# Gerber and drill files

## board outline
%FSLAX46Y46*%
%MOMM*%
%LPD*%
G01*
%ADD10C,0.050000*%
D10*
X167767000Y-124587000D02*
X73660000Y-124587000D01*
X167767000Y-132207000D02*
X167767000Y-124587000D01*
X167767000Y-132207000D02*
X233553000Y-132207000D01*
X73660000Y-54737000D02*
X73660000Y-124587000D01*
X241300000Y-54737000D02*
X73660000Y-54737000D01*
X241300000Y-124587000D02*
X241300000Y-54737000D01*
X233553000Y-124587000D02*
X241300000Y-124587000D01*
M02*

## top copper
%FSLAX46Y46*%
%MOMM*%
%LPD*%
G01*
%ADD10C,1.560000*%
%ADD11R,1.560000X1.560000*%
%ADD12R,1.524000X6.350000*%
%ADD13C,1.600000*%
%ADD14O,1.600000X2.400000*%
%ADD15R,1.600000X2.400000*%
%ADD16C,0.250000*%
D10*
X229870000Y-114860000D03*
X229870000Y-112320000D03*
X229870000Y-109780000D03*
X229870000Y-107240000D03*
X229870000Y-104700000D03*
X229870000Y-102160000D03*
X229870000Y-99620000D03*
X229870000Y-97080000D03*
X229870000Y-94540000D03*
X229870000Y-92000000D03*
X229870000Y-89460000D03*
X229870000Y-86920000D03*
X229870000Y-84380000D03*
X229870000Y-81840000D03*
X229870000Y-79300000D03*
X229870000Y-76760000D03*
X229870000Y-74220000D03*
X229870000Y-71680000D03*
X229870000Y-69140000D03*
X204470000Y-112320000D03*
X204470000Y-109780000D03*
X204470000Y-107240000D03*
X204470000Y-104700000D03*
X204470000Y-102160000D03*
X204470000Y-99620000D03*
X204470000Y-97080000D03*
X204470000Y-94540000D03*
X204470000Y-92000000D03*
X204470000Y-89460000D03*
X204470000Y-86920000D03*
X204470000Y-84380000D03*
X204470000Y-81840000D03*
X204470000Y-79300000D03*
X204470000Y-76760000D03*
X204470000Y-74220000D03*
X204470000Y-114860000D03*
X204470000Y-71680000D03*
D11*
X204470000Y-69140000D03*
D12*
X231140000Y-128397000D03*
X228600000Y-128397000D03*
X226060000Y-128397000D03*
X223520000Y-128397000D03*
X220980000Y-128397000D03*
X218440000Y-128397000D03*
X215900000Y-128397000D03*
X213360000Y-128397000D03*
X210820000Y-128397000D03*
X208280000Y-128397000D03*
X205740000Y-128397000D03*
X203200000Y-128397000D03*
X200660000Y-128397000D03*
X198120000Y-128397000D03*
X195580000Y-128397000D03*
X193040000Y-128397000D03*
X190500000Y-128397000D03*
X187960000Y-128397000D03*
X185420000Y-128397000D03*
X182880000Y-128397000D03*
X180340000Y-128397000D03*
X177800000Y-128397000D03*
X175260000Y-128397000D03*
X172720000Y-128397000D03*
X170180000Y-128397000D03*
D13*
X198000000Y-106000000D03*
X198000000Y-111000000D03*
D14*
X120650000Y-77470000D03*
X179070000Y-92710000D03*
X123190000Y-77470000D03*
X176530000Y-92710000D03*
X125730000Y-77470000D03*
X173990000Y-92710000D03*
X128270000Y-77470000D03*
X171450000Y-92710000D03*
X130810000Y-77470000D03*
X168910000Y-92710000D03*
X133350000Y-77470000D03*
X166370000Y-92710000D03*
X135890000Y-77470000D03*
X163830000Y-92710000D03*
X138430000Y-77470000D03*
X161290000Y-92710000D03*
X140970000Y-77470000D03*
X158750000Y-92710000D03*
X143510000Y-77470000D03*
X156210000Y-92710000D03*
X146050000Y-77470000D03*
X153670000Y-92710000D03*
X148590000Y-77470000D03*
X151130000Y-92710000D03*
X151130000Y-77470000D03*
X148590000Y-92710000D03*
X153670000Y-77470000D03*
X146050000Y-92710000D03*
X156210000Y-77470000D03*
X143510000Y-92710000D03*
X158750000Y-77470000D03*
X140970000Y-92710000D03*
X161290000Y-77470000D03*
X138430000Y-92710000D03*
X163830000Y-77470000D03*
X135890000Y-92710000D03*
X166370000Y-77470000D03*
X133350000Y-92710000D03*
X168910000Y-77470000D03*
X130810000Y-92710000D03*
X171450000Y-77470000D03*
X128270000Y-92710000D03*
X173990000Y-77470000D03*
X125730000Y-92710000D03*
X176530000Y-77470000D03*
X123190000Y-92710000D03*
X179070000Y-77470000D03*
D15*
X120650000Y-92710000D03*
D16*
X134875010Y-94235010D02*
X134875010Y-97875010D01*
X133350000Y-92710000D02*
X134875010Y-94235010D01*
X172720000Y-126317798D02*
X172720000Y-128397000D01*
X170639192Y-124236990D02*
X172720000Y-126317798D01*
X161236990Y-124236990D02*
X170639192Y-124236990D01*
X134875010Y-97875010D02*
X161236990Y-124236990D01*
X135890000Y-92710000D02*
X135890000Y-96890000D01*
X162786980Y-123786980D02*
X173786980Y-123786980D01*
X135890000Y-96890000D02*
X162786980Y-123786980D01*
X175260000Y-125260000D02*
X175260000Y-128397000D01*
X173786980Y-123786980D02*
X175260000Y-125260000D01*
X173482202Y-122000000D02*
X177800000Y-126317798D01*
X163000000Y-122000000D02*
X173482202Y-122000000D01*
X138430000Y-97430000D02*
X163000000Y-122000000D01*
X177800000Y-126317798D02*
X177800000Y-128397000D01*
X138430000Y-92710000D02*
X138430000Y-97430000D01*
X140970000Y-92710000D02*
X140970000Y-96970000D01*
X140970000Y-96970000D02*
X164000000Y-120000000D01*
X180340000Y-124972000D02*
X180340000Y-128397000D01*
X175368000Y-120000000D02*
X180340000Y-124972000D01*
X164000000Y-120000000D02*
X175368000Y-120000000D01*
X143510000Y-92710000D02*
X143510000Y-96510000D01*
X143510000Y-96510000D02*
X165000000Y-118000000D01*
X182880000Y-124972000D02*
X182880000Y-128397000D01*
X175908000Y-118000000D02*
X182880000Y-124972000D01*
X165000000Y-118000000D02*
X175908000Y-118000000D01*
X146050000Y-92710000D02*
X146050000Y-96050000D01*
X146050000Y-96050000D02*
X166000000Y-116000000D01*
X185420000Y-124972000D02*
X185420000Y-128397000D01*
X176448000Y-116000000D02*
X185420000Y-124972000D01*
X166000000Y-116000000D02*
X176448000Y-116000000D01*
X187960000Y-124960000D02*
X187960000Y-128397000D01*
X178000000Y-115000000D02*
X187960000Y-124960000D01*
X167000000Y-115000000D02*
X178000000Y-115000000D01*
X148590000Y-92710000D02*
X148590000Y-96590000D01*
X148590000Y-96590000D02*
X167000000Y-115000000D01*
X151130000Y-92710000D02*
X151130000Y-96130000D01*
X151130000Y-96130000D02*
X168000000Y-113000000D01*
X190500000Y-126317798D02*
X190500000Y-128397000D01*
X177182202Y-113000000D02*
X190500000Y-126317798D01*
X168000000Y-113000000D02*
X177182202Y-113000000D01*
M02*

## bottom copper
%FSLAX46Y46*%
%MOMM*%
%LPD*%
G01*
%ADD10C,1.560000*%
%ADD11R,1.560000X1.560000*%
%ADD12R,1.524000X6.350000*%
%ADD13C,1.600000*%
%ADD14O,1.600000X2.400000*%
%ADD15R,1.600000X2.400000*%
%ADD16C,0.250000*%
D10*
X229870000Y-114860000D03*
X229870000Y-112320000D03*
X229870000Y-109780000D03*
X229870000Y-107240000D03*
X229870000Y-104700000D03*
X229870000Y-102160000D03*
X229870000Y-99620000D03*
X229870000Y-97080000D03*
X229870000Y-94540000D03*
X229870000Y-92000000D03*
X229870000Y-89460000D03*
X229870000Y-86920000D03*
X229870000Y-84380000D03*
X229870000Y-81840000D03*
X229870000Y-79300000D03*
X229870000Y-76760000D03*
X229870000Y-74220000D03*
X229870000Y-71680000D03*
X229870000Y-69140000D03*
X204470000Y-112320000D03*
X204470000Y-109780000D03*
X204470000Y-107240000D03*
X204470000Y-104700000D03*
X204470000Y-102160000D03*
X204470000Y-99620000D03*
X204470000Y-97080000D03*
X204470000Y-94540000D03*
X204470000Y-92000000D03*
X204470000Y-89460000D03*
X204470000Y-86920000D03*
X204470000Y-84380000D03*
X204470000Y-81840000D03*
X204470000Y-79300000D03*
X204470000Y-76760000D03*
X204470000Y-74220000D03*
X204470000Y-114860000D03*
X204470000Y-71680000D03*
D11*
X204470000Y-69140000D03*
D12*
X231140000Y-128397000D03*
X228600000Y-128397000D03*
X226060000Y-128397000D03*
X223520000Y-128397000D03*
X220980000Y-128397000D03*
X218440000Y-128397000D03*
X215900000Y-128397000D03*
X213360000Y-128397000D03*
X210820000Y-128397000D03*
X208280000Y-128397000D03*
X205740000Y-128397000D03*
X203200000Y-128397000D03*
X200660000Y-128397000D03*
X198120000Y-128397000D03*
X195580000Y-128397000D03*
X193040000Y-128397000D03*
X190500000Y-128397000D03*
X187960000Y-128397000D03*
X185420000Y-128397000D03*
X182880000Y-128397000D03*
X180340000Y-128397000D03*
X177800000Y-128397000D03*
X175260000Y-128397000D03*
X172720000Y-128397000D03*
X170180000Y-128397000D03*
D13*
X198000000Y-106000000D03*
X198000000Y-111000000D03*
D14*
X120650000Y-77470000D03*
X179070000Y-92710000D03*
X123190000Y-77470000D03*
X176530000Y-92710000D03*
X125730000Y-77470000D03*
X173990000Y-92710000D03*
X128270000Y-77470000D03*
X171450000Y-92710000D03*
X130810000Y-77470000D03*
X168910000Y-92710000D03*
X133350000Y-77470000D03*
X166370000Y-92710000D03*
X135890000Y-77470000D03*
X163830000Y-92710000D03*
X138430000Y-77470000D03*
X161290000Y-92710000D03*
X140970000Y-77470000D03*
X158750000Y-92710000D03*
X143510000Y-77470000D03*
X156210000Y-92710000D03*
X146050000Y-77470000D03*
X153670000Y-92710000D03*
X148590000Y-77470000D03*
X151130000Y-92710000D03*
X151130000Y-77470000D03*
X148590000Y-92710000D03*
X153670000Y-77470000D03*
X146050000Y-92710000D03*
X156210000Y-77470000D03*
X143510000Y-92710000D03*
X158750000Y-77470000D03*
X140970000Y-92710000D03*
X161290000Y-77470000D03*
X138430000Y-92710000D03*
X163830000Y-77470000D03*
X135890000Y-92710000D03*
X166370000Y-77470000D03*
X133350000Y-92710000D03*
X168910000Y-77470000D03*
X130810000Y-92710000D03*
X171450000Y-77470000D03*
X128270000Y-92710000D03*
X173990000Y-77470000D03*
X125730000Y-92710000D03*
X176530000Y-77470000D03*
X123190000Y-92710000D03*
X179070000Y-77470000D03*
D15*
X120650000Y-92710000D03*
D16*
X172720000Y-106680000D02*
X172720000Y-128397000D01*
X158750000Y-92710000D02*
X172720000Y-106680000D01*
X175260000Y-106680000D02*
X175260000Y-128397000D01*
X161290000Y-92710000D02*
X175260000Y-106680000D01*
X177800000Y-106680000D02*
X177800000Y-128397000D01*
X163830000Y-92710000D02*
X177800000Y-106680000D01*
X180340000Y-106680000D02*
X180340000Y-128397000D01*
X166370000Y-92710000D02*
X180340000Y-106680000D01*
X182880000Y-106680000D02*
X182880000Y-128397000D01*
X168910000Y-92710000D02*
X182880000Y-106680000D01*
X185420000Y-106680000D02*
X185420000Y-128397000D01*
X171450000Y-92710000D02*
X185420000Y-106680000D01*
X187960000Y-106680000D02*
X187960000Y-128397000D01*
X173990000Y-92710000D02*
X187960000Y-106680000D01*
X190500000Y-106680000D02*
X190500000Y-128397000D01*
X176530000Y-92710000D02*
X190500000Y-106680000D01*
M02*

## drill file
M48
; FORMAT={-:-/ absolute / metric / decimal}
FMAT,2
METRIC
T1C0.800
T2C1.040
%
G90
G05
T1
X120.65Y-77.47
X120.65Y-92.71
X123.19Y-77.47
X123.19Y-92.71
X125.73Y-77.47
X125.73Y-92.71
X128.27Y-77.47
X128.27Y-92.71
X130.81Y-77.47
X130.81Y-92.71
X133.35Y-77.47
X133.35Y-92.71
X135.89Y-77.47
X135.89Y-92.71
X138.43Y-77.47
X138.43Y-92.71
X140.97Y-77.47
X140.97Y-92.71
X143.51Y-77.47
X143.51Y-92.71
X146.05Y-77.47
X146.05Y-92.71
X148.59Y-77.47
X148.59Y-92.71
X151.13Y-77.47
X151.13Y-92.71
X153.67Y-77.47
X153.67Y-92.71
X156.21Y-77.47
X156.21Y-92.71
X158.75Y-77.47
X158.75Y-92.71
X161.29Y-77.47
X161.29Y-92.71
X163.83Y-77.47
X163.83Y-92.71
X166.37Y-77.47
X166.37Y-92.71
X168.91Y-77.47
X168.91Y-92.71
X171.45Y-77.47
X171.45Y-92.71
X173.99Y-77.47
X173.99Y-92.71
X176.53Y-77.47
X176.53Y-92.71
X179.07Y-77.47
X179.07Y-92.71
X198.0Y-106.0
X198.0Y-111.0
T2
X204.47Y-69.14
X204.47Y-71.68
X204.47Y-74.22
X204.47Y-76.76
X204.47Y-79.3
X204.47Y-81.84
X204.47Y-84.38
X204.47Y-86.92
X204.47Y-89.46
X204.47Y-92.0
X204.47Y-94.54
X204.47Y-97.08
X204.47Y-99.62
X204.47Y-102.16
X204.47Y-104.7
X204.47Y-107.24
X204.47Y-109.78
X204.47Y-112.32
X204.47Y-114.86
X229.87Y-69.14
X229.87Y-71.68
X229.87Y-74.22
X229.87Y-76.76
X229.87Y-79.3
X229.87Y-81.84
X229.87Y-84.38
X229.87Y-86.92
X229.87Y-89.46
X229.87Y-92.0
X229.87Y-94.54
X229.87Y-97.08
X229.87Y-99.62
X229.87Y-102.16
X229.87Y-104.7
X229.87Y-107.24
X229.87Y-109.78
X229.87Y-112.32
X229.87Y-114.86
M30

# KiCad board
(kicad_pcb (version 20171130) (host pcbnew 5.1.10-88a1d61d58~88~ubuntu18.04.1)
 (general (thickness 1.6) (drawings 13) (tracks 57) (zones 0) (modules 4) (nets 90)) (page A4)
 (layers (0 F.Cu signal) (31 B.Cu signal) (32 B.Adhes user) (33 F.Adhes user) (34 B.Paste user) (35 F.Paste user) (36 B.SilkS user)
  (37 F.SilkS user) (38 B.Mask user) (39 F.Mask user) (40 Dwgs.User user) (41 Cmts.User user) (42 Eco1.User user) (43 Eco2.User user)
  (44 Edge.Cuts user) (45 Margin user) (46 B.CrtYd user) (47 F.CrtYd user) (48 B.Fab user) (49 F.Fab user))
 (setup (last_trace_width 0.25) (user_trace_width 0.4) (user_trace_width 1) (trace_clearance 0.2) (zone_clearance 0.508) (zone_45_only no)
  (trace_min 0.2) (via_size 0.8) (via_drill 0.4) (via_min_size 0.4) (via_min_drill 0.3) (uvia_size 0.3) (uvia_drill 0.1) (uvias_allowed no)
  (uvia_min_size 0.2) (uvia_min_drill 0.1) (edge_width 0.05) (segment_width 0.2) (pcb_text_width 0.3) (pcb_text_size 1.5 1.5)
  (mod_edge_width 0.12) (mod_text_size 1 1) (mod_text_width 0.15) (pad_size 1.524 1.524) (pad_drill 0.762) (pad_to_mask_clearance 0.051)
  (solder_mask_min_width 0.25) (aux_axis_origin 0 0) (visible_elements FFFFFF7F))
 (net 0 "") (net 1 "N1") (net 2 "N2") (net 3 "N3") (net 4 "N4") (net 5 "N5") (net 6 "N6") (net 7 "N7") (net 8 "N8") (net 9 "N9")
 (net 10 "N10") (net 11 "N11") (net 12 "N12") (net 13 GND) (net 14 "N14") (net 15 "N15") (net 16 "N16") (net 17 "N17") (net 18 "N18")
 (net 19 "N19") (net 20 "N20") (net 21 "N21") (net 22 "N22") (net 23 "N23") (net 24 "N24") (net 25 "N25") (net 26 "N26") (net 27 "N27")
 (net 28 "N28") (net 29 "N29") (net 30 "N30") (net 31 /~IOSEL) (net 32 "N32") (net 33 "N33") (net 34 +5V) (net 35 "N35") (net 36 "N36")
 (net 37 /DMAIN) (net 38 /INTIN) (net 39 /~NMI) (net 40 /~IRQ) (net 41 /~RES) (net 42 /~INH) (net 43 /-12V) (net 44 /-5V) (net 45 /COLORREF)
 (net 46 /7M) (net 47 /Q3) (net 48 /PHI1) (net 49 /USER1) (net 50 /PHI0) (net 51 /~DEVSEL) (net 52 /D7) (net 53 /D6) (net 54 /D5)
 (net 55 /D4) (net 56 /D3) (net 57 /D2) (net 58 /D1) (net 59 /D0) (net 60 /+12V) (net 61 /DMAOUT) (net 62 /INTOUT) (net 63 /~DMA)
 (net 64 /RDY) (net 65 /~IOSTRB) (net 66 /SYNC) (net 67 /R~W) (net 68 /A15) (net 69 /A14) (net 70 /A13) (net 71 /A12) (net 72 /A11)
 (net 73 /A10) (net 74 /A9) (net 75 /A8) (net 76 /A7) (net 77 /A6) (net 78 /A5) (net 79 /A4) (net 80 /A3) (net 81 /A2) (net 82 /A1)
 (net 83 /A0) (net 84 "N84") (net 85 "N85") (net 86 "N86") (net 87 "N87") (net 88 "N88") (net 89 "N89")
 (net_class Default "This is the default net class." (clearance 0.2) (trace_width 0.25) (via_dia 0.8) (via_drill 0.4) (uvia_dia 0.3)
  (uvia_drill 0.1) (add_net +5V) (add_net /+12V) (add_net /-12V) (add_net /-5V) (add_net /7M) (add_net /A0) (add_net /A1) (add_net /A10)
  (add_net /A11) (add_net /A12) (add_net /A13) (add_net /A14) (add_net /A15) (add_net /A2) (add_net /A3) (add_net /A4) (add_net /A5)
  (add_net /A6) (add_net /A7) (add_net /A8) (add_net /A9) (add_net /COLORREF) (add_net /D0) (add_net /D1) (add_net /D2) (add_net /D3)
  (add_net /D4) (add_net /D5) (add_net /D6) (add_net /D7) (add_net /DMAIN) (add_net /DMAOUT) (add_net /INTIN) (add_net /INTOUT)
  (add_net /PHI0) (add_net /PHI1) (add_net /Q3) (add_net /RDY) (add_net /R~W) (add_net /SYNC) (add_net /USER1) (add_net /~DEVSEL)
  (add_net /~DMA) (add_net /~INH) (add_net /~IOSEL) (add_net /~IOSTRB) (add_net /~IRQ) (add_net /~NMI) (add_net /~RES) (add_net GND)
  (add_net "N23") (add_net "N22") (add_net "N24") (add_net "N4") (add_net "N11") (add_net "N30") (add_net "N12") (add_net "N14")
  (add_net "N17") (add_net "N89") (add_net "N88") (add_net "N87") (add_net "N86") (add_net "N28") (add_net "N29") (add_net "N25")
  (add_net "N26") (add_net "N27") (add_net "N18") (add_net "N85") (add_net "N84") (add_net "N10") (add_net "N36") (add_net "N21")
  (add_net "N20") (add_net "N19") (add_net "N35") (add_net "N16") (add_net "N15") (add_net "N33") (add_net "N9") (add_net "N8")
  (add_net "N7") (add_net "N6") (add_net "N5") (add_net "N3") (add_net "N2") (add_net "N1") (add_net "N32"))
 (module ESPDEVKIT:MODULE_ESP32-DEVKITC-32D (layer F.Cu) (at 217.17 88.9)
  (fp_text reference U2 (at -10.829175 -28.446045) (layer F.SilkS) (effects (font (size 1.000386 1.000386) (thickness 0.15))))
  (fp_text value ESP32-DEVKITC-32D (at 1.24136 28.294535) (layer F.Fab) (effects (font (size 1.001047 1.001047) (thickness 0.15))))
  (pad 38 thru_hole circle (at 12.7 25.96) (size 1.56 1.56) (drill 1.04) (layers *.Cu *.Mask) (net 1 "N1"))
  (pad 37 thru_hole circle (at 12.7 23.42) (size 1.56 1.56) (drill 1.04) (layers *.Cu *.Mask) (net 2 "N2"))
  (pad 36 thru_hole circle (at 12.7 20.88) (size 1.56 1.56) (drill 1.04) (layers *.Cu *.Mask) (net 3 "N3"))
  (pad 35 thru_hole circle (at 12.7 18.34) (size 1.56 1.56) (drill 1.04) (layers *.Cu *.Mask) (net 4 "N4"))
  (pad 34 thru_hole circle (at 12.7 15.8) (size 1.56 1.56) (drill 1.04) (layers *.Cu *.Mask) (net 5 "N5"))
  (pad 33 thru_hole circle (at 12.7 13.26) (size 1.56 1.56) (drill 1.04) (layers *.Cu *.Mask) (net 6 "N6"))
  (pad 32 thru_hole circle (at 12.7 10.72) (size 1.56 1.56) (drill 1.04) (layers *.Cu *.Mask) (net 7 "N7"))
  (pad 31 thru_hole circle (at 12.7 8.18) (size 1.56 1.56) (drill 1.04) (layers *.Cu *.Mask) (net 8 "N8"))
  (pad 30 thru_hole circle (at 12.7 5.64) (size 1.56 1.56) (drill 1.04) (layers *.Cu *.Mask) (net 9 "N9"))
  (pad 29 thru_hole circle (at 12.7 3.1) (size 1.56 1.56) (drill 1.04) (layers *.Cu *.Mask) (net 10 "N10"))
  (pad 28 thru_hole circle (at 12.7 0.56) (size 1.56 1.56) (drill 1.04) (layers *.Cu *.Mask) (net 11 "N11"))
  (pad 27 thru_hole circle (at 12.7 -1.98) (size 1.56 1.56) (drill 1.04) (layers *.Cu *.Mask) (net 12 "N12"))
  (pad 26 thru_hole circle (at 12.7 -4.52) (size 1.56 1.56) (drill 1.04) (layers *.Cu *.Mask) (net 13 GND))
  (pad 25 thru_hole circle (at 12.7 -7.06) (size 1.56 1.56) (drill 1.04) (layers *.Cu *.Mask) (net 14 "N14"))
  (pad 24 thru_hole circle (at 12.7 -9.6) (size 1.56 1.56) (drill 1.04) (layers *.Cu *.Mask) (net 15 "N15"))
  (pad 23 thru_hole circle (at 12.7 -12.14) (size 1.56 1.56) (drill 1.04) (layers *.Cu *.Mask) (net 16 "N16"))
  (pad 22 thru_hole circle (at 12.7 -14.68) (size 1.56 1.56) (drill 1.04) (layers *.Cu *.Mask) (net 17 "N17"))
  (pad 21 thru_hole circle (at 12.7 -17.22) (size 1.56 1.56) (drill 1.04) (layers *.Cu *.Mask) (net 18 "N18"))
  (pad 20 thru_hole circle (at 12.7 -19.76) (size 1.56 1.56) (drill 1.04) (layers *.Cu *.Mask) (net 13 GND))
  (pad 18 thru_hole circle (at -12.7 23.42) (size 1.56 1.56) (drill 1.04) (layers *.Cu *.Mask) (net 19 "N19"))
  (pad 17 thru_hole circle (at -12.7 20.88) (size 1.56 1.56) (drill 1.04) (layers *.Cu *.Mask) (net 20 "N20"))
  (pad 16 thru_hole circle (at -12.7 18.34) (size 1.56 1.56) (drill 1.04) (layers *.Cu *.Mask) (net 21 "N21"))
  (pad 15 thru_hole circle (at -12.7 15.8) (size 1.56 1.56) (drill 1.04) (layers *.Cu *.Mask) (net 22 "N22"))
  (pad 14 thru_hole circle (at -12.7 13.26) (size 1.56 1.56) (drill 1.04) (layers *.Cu *.Mask) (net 13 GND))
  (pad 13 thru_hole circle (at -12.7 10.72) (size 1.56 1.56) (drill 1.04) (layers *.Cu *.Mask) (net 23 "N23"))
  (pad 12 thru_hole circle (at -12.7 8.18) (size 1.56 1.56) (drill 1.04) (layers *.Cu *.Mask) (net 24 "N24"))
  (pad 11 thru_hole circle (at -12.7 5.64) (size 1.56 1.56) (drill 1.04) (layers *.Cu *.Mask) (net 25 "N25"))
  (pad 10 thru_hole circle (at -12.7 3.1) (size 1.56 1.56) (drill 1.04) (layers *.Cu *.Mask) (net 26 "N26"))
  (pad 9 thru_hole circle (at -12.7 0.56) (size 1.56 1.56) (drill 1.04) (layers *.Cu *.Mask) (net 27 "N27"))
  (pad 8 thru_hole circle (at -12.7 -1.98) (size 1.56 1.56) (drill 1.04) (layers *.Cu *.Mask) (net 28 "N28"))
  (pad 7 thru_hole circle (at -12.7 -4.52) (size 1.56 1.56) (drill 1.04) (layers *.Cu *.Mask) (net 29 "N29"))
  (pad 6 thru_hole circle (at -12.7 -7.06) (size 1.56 1.56) (drill 1.04) (layers *.Cu *.Mask) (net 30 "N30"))
  (pad 5 thru_hole circle (at -12.7 -9.6) (size 1.56 1.56) (drill 1.04) (layers *.Cu *.Mask) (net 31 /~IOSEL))
  (pad 4 thru_hole circle (at -12.7 -12.14) (size 1.56 1.56) (drill 1.04) (layers *.Cu *.Mask) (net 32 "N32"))
  (pad 3 thru_hole circle (at -12.7 -14.68) (size 1.56 1.56) (drill 1.04) (layers *.Cu *.Mask) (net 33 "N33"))
  (pad 19 thru_hole circle (at -12.7 25.96) (size 1.56 1.56) (drill 1.04) (layers *.Cu *.Mask) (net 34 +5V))
  (pad 2 thru_hole circle (at -12.7 -17.22) (size 1.56 1.56) (drill 1.04) (layers *.Cu *.Mask) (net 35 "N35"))
  (pad 1 thru_hole rect (at -12.7 -19.76) (size 1.56 1.56) (drill 1.04) (layers *.Cu *.Mask) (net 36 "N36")))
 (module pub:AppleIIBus (layer F.Cu) (at 200.66 128.397)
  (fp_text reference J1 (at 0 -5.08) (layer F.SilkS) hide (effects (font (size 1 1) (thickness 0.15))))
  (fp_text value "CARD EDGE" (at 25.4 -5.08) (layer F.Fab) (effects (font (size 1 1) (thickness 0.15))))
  (pad 26 smd rect (at 30.48 0) (size 1.524 6.35) (layers B.Cu B.Mask) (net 13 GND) (solder_mask_margin 0.635) (clearance 0.254))
  (pad 27 smd rect (at 27.94 0) (size 1.524 6.35) (layers B.Cu B.Mask) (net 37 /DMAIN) (solder_mask_margin 0.635) (clearance 0.254))
  (pad 28 smd rect (at 25.4 0) (size 1.524 6.35) (layers B.Cu B.Mask) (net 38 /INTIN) (solder_mask_margin 0.635) (clearance 0.254))
  (pad 29 smd rect (at 22.86 0) (size 1.524 6.35) (layers B.Cu B.Mask) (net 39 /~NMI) (solder_mask_margin 0.635) (clearance 0.254))
  (pad 30 smd rect (at 20.32 0) (size 1.524 6.35) (layers B.Cu B.Mask) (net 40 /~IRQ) (solder_mask_margin 0.635) (clearance 0.254))
  (pad 31 smd rect (at 17.78 0) (size 1.524 6.35) (layers B.Cu B.Mask) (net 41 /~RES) (solder_mask_margin 0.635) (clearance 0.254))
  (pad 32 smd rect (at 15.24 0) (size 1.524 6.35) (layers B.Cu B.Mask) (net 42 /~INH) (solder_mask_margin 0.635) (clearance 0.254))
  (pad 33 smd rect (at 12.7 0) (size 1.524 6.35) (layers B.Cu B.Mask) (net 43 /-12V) (solder_mask_margin 0.635) (clearance 0.254))
  (pad 34 smd rect (at 10.16 0) (size 1.524 6.35) (layers B.Cu B.Mask) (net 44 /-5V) (solder_mask_margin 0.635) (clearance 0.254))
  (pad 35 smd rect (at 7.62 0) (size 1.524 6.35) (layers B.Cu B.Mask) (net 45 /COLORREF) (solder_mask_margin 0.635) (clearance 0.254))
  (pad 36 smd rect (at 5.08 0) (size 1.524 6.35) (layers B.Cu B.Mask) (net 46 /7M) (solder_mask_margin 0.635) (clearance 0.254))
  (pad 37 smd rect (at 2.54 0) (size 1.524 6.35) (layers B.Cu B.Mask) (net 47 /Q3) (solder_mask_margin 0.635) (clearance 0.254))
  (pad 38 smd rect (at 0 0) (size 1.524 6.35) (layers B.Cu B.Mask) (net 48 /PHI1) (solder_mask_margin 0.635) (clearance 0.254))
  (pad 39 smd rect (at -2.54 0) (size 1.524 6.35) (layers B.Cu B.Mask) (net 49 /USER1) (solder_mask_margin 0.635) (clearance 0.254))
  (pad 40 smd rect (at -5.08 0) (size 1.524 6.35) (layers B.Cu B.Mask) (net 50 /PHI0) (solder_mask_margin 0.635) (clearance 0.254))
  (pad 41 smd rect (at -7.62 0) (size 1.524 6.35) (layers B.Cu B.Mask) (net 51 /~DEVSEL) (solder_mask_margin 0.635) (clearance 0.254))
  (pad 42 smd rect (at -10.16 0) (size 1.524 6.35) (layers B.Cu B.Mask) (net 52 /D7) (solder_mask_margin 0.635) (clearance 0.254))
  (pad 43 smd rect (at -12.7 0) (size 1.524 6.35) (layers B.Cu B.Mask) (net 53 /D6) (solder_mask_margin 0.635) (clearance 0.254))
  (pad 44 smd rect (at -15.24 0) (size 1.524 6.35) (layers B.Cu B.Mask) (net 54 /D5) (solder_mask_margin 0.635) (clearance 0.254))
  (pad 45 smd rect (at -17.78 0) (size 1.524 6.35) (layers B.Cu B.Mask) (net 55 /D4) (solder_mask_margin 0.635) (clearance 0.254))
  (pad 46 smd rect (at -20.32 0) (size 1.524 6.35) (layers B.Cu B.Mask) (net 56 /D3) (solder_mask_margin 0.635) (clearance 0.254))
  (pad 47 smd rect (at -22.86 0) (size 1.524 6.35) (layers B.Cu B.Mask) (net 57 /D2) (solder_mask_margin 0.635) (clearance 0.254))
  (pad 48 smd rect (at -25.4 0) (size 1.524 6.35) (layers B.Cu B.Mask) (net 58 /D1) (solder_mask_margin 0.635) (clearance 0.254))
  (pad 49 smd rect (at -27.94 0) (size 1.524 6.35) (layers B.Cu B.Mask) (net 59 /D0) (solder_mask_margin 0.635) (clearance 0.254))
  (pad 50 smd rect (at -30.48 0) (size 1.524 6.35) (layers B.Cu B.Mask) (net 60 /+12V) (solder_mask_margin 0.635) (clearance 0.254))
  (pad 25 smd rect (at 30.48 0) (size 1.524 6.35) (layers F.Cu F.Mask) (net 34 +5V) (solder_mask_margin 0.635) (clearance 0.254))
  (pad 24 smd rect (at 27.94 0) (size 1.524 6.35) (layers F.Cu F.Mask) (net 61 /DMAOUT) (solder_mask_margin 0.635) (clearance 0.254))
  (pad 23 smd rect (at 25.4 0) (size 1.524 6.35) (layers F.Cu F.Mask) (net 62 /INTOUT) (solder_mask_margin 0.635) (clearance 0.254))
  (pad 22 smd rect (at 22.86 0) (size 1.524 6.35) (layers F.Cu F.Mask) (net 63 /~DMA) (solder_mask_margin 0.635) (clearance 0.254))
  (pad 21 smd rect (at 20.32 0) (size 1.524 6.35) (layers F.Cu F.Mask) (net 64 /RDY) (solder_mask_margin 0.635) (clearance 0.254))
  (pad 20 smd rect (at 17.78 0) (size 1.524 6.35) (layers F.Cu F.Mask) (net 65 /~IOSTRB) (solder_mask_margin 0.635) (clearance 0.254))
  (pad 19 smd rect (at 15.24 0) (size 1.524 6.35) (layers F.Cu F.Mask) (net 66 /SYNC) (solder_mask_margin 0.635) (clearance 0.254))
  (pad 18 smd rect (at 12.7 0) (size 1.524 6.35) (layers F.Cu F.Mask) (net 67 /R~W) (solder_mask_margin 0.635) (clearance 0.254))
  (pad 17 smd rect (at 10.16 0) (size 1.524 6.35) (layers F.Cu F.Mask) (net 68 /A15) (solder_mask_margin 0.635) (clearance 0.254))
  (pad 16 smd rect (at 7.62 0) (size 1.524 6.35) (layers F.Cu F.Mask) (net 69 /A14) (solder_mask_margin 0.635) (clearance 0.254))
  (pad 15 smd rect (at 5.08 0) (size 1.524 6.35) (layers F.Cu F.Mask) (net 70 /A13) (solder_mask_margin 0.635) (clearance 0.254))
  (pad 14 smd rect (at 2.54 0) (size 1.524 6.35) (layers F.Cu F.Mask) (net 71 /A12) (solder_mask_margin 0.635) (clearance 0.254))
  (pad 13 smd rect (at 0 0) (size 1.524 6.35) (layers F.Cu F.Mask) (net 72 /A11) (solder_mask_margin 0.635) (clearance 0.254))
  (pad 12 smd rect (at -2.54 0) (size 1.524 6.35) (layers F.Cu F.Mask) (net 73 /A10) (solder_mask_margin 0.635) (clearance 0.254))
  (pad 11 smd rect (at -5.08 0) (size 1.524 6.35) (layers F.Cu F.Mask) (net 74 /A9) (solder_mask_margin 0.635) (clearance 0.254))
  (pad 10 smd rect (at -7.62 0) (size 1.524 6.35) (layers F.Cu F.Mask) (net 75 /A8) (solder_mask_margin 0.635) (clearance 0.254))
  (pad 9 smd rect (at -10.16 0) (size 1.524 6.35) (layers F.Cu F.Mask) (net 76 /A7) (solder_mask_margin 0.635) (clearance 0.254))
  (pad 8 smd rect (at -12.7 0) (size 1.524 6.35) (layers F.Cu F.Mask) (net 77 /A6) (solder_mask_margin 0.635) (clearance 0.254))
  (pad 7 smd rect (at -15.24 0) (size 1.524 6.35) (layers F.Cu F.Mask) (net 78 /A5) (solder_mask_margin 0.635) (clearance 0.254))
  (pad 6 smd rect (at -17.78 0) (size 1.524 6.35) (layers F.Cu F.Mask) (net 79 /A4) (solder_mask_margin 0.635) (clearance 0.254))
  (pad 5 smd rect (at -20.32 0) (size 1.524 6.35) (layers F.Cu F.Mask) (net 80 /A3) (solder_mask_margin 0.635) (clearance 0.254))
  (pad 4 smd rect (at -22.86 0) (size 1.524 6.35) (layers F.Cu F.Mask) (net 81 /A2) (solder_mask_margin 0.635) (clearance 0.254))
  (pad 3 smd rect (at -25.4 0) (size 1.524 6.35) (layers F.Cu F.Mask) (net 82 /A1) (solder_mask_margin 0.635) (clearance 0.254))
  (pad 2 smd rect (at -27.94 0) (size 1.524 6.35) (layers F.Cu F.Mask) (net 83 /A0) (solder_mask_margin 0.635) (clearance 0.254))
  (pad 1 smd rect (at -30.48 0) (size 1.524 6.35) (layers F.Cu F.Mask) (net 31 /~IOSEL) (solder_mask_margin 0.635) (clearance 0.254)))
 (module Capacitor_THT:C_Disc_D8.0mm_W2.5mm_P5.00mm (layer F.Cu) (at 198 111 90)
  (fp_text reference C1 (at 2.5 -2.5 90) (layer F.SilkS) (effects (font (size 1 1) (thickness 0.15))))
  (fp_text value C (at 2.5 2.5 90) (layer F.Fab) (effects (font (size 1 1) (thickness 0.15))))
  (pad 2 thru_hole circle (at 5 0 90) (size 1.6 1.6) (drill 0.8) (layers *.Cu *.Mask) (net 13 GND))
  (pad 1 thru_hole circle (at 0 0 90) (size 1.6 1.6) (drill 0.8) (layers *.Cu *.Mask) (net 34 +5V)))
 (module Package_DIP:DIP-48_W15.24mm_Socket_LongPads (layer F.Cu) (at 120.65 92.71 90)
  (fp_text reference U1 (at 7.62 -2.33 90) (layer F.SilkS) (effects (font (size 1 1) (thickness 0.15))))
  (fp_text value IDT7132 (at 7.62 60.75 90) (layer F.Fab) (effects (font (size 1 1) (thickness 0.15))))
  (pad 48 thru_hole oval (at 15.24 0 90) (size 2.4 1.6) (drill 0.8) (layers *.Cu *.Mask) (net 34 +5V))
  (pad 24 thru_hole oval (at 0 58.42 90) (size 2.4 1.6) (drill 0.8) (layers *.Cu *.Mask) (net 13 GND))
  (pad 47 thru_hole oval (at 15.24 2.54 90) (size 2.4 1.6) (drill 0.8) (layers *.Cu *.Mask) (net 13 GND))
  (pad 23 thru_hole oval (at 0 55.88 90) (size 2.4 1.6) (drill 0.8) (layers *.Cu *.Mask) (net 52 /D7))
  (pad 46 thru_hole oval (at 15.24 5.08 90) (size 2.4 1.6) (drill 0.8) (layers *.Cu *.Mask) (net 10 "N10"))
  (pad 22 thru_hole oval (at 0 53.34 90) (size 2.4 1.6) (drill 0.8) (layers *.Cu *.Mask) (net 53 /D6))
  (pad 45 thru_hole oval (at 15.24 7.62 90) (size 2.4 1.6) (drill 0.8) (layers *.Cu *.Mask) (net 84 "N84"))
  (pad 21 thru_hole oval (at 0 50.8 90) (size 2.4 1.6) (drill 0.8) (layers *.Cu *.Mask) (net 54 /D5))
  (pad 44 thru_hole oval (at 15.24 10.16 90) (size 2.4 1.6) (drill 0.8) (layers *.Cu *.Mask) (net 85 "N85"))
  (pad 20 thru_hole oval (at 0 48.26 90) (size 2.4 1.6) (drill 0.8) (layers *.Cu *.Mask) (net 55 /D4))
  (pad 43 thru_hole oval (at 15.24 12.7 90) (size 2.4 1.6) (drill 0.8) (layers *.Cu *.Mask) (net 13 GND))
  (pad 19 thru_hole oval (at 0 45.72 90) (size 2.4 1.6) (drill 0.8) (layers *.Cu *.Mask) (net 56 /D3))
  (pad 42 thru_hole oval (at 15.24 15.24 90) (size 2.4 1.6) (drill 0.8) (layers *.Cu *.Mask) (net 18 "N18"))
  (pad 18 thru_hole oval (at 0 43.18 90) (size 2.4 1.6) (drill 0.8) (layers *.Cu *.Mask) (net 57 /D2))
  (pad 41 thru_hole oval (at 15.24 17.78 90) (size 2.4 1.6) (drill 0.8) (layers *.Cu *.Mask) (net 27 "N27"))
  (pad 17 thru_hole oval (at 0 40.64 90) (size 2.4 1.6) (drill 0.8) (layers *.Cu *.Mask) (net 58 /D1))
  (pad 40 thru_hole oval (at 15.24 20.32 90) (size 2.4 1.6) (drill 0.8) (layers *.Cu *.Mask) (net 26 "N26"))
  (pad 16 thru_hole oval (at 0 38.1 90) (size 2.4 1.6) (drill 0.8) (layers *.Cu *.Mask) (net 59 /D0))
  (pad 39 thru_hole oval (at 15.24 22.86 90) (size 2.4 1.6) (drill 0.8) (layers *.Cu *.Mask) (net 25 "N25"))
  (pad 15 thru_hole oval (at 0 35.56 90) (size 2.4 1.6) (drill 0.8) (layers *.Cu *.Mask) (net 13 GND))
  (pad 38 thru_hole oval (at 15.24 25.4 90) (size 2.4 1.6) (drill 0.8) (layers *.Cu *.Mask) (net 29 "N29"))
  (pad 14 thru_hole oval (at 0 33.02 90) (size 2.4 1.6) (drill 0.8) (layers *.Cu *.Mask) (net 13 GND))
  (pad 37 thru_hole oval (at 15.24 27.94 90) (size 2.4 1.6) (drill 0.8) (layers *.Cu *.Mask) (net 28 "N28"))
  (pad 13 thru_hole oval (at 0 30.48 90) (size 2.4 1.6) (drill 0.8) (layers *.Cu *.Mask) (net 76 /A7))
  (pad 36 thru_hole oval (at 15.24 30.48 90) (size 2.4 1.6) (drill 0.8) (layers *.Cu *.Mask) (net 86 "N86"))
  (pad 12 thru_hole oval (at 0 27.94 90) (size 2.4 1.6) (drill 0.8) (layers *.Cu *.Mask) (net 77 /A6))
  (pad 35 thru_hole oval (at 15.24 33.02 90) (size 2.4 1.6) (drill 0.8) (layers *.Cu *.Mask) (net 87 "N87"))
  (pad 11 thru_hole oval (at 0 25.4 90) (size 2.4 1.6) (drill 0.8) (layers *.Cu *.Mask) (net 78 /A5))
  (pad 34 thru_hole oval (at 15.24 35.56 90) (size 2.4 1.6) (drill 0.8) (layers *.Cu *.Mask) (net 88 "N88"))
  (pad 10 thru_hole oval (at 0 22.86 90) (size 2.4 1.6) (drill 0.8) (layers *.Cu *.Mask) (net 79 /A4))
  (pad 33 thru_hole oval (at 15.24 38.1 90) (size 2.4 1.6) (drill 0.8) (layers *.Cu *.Mask) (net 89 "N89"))
  (pad 9 thru_hole oval (at 0 20.32 90) (size 2.4 1.6) (drill 0.8) (layers *.Cu *.Mask) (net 80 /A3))
  (pad 32 thru_hole oval (at 15.24 40.64 90) (size 2.4 1.6) (drill 0.8) (layers *.Cu *.Mask) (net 17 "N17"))
  (pad 8 thru_hole oval (at 0 17.78 90) (size 2.4 1.6) (drill 0.8) (layers *.Cu *.Mask) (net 81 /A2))
  (pad 31 thru_hole oval (at 15.24 43.18 90) (size 2.4 1.6) (drill 0.8) (layers *.Cu *.Mask) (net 14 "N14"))
  (pad 7 thru_hole oval (at 0 15.24 90) (size 2.4 1.6) (drill 0.8) (layers *.Cu *.Mask) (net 82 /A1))
  (pad 30 thru_hole oval (at 15.24 45.72 90) (size 2.4 1.6) (drill 0.8) (layers *.Cu *.Mask) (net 12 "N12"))
  (pad 6 thru_hole oval (at 0 12.7 90) (size 2.4 1.6) (drill 0.8) (layers *.Cu *.Mask) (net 83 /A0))
  (pad 29 thru_hole oval (at 15.24 48.26 90) (size 2.4 1.6) (drill 0.8) (layers *.Cu *.Mask) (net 11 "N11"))
  (pad 5 thru_hole oval (at 0 10.16 90) (size 2.4 1.6) (drill 0.8) (layers *.Cu *.Mask) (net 13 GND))
  (pad 28 thru_hole oval (at 15.24 50.8 90) (size 2.4 1.6) (drill 0.8) (layers *.Cu *.Mask) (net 4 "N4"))
  (pad 4 thru_hole oval (at 0 7.62 90) (size 2.4 1.6) (drill 0.8) (layers *.Cu *.Mask) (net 13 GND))
  (pad 27 thru_hole oval (at 15.24 53.34 90) (size 2.4 1.6) (drill 0.8) (layers *.Cu *.Mask) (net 24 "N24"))
  (pad 3 thru_hole oval (at 0 5.08 90) (size 2.4 1.6) (drill 0.8) (layers *.Cu *.Mask) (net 30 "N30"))
  (pad 26 thru_hole oval (at 15.24 55.88 90) (size 2.4 1.6) (drill 0.8) (layers *.Cu *.Mask) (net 22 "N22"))
  (pad 2 thru_hole oval (at 0 2.54 90) (size 2.4 1.6) (drill 0.8) (layers *.Cu *.Mask) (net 67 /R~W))
  (pad 25 thru_hole oval (at 15.24 58.42 90) (size 2.4 1.6) (drill 0.8) (layers *.Cu *.Mask) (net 23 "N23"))
  (pad 1 thru_hole rect (at 0 0 90) (size 2.4 1.6) (drill 0.8) (layers *.Cu *.Mask) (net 51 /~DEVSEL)))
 (gr_line (start 167.767 124.587) (end 73.66 124.587) (layer Edge.Cuts) (width 0.05))
 (gr_line (start 167.767 132.207) (end 167.767 124.587) (layer Edge.Cuts) (width 0.05))
 (gr_line (start 167.767 132.207) (end 233.553 132.207) (layer Edge.Cuts) (width 0.05))
 (gr_line (start 73.66 54.737) (end 73.66 124.587) (layer Edge.Cuts) (width 0.05))
 (gr_line (start 241.3 54.737) (end 73.66 54.737) (layer Edge.Cuts) (width 0.05))
 (gr_line (start 241.3 124.587) (end 241.3 54.737) (layer Edge.Cuts) (width 0.05))
 (gr_line (start 233.553 124.587) (end 241.3 124.587) (layer Edge.Cuts) (width 0.05))
 (segment (start 172.72 106.68) (end 172.72 128.397) (width 0.25) (layer B.Cu) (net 59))
 (segment (start 158.75 92.71) (end 172.72 106.68) (width 0.25) (layer B.Cu) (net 59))
 (segment (start 175.26 106.68) (end 175.26 128.397) (width 0.25) (layer B.Cu) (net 58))
 (segment (start 161.29 92.71) (end 175.26 106.68) (width 0.25) (layer B.Cu) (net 58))
 (segment (start 177.8 106.68) (end 177.8 128.397) (width 0.25) (layer B.Cu) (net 57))
 (segment (start 163.83 92.71) (end 177.8 106.68) (width 0.25) (layer B.Cu) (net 57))
 (segment (start 180.34 106.68) (end 180.34 128.397) (width 0.25) (layer B.Cu) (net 56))
 (segment (start 166.37 92.71) (end 180.34 106.68) (width 0.25) (layer B.Cu) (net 56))
 (segment (start 182.88 106.68) (end 182.88 128.397) (width 0.25) (layer B.Cu) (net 55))
 (segment (start 168.91 92.71) (end 182.88 106.68) (width 0.25) (layer B.Cu) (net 55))
 (segment (start 185.42 106.68) (end 185.42 128.397) (width 0.25) (layer B.Cu) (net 54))
 (segment (start 171.45 92.71) (end 185.42 106.68) (width 0.25) (layer B.Cu) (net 54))
 (segment (start 187.96 106.68) (end 187.96 128.397) (width 0.25) (layer B.Cu) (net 53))
 (segment (start 173.99 92.71) (end 187.96 106.68) (width 0.25) (layer B.Cu) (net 53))
 (segment (start 190.5 106.68) (end 190.5 128.397) (width 0.25) (layer B.Cu) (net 52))
 (segment (start 176.53 92.71) (end 190.5 106.68) (width 0.25) (layer B.Cu) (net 52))
 (segment (start 134.87501 94.23501) (end 134.87501 97.87501) (width 0.25) (layer F.Cu) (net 83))
 (segment (start 133.35 92.71) (end 134.87501 94.23501) (width 0.25) (layer F.Cu) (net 83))
 (segment (start 172.72 126.317798) (end 172.72 128.397) (width 0.25) (layer F.Cu) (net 83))
 (segment (start 170.639192 124.23699) (end 172.72 126.317798) (width 0.25) (layer F.Cu) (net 83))
 (segment (start 161.23699 124.23699) (end 170.639192 124.23699) (width 0.25) (layer F.Cu) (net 83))
 (segment (start 134.87501 97.87501) (end 161.23699 124.23699) (width 0.25) (layer F.Cu) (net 83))
 (segment (start 135.89 92.71) (end 135.89 96.89) (width 0.25) (layer F.Cu) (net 82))
 (segment (start 162.78698 123.78698) (end 173.78698 123.78698) (width 0.25) (layer F.Cu) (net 82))
 (segment (start 135.89 96.89) (end 162.78698 123.78698) (width 0.25) (layer F.Cu) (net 82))
 (segment (start 175.26 125.26) (end 175.26 128.397) (width 0.25) (layer F.Cu) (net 82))
 (segment (start 173.78698 123.78698) (end 175.26 125.26) (width 0.25) (layer F.Cu) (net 82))
 (segment (start 173.482202 122) (end 177.8 126.317798) (width 0.25) (layer F.Cu) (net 81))
 (segment (start 163 122) (end 173.482202 122) (width 0.25) (layer F.Cu) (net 81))
 (segment (start 138.43 97.43) (end 163 122) (width 0.25) (layer F.Cu) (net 81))
 (segment (start 177.8 126.317798) (end 177.8 128.397) (width 0.25) (layer F.Cu) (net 81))
 (segment (start 138.43 92.71) (end 138.43 97.43) (width 0.25) (layer F.Cu) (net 81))
 (segment (start 140.97 92.71) (end 140.97 96.97) (width 0.25) (layer F.Cu) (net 80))
 (segment (start 140.97 96.97) (end 164 120) (width 0.25) (layer F.Cu) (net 80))
 (segment (start 180.34 124.972) (end 180.34 128.397) (width 0.25) (layer F.Cu) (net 80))
 (segment (start 175.368 120) (end 180.34 124.972) (width 0.25) (layer F.Cu) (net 80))
 (segment (start 164 120) (end 175.368 120) (width 0.25) (layer F.Cu) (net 80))
 (segment (start 143.51 92.71) (end 143.51 96.51) (width 0.25) (layer F.Cu) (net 79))
 (segment (start 143.51 96.51) (end 165 118) (width 0.25) (layer F.Cu) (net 79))
 (segment (start 182.88 124.972) (end 182.88 128.397) (width 0.25) (layer F.Cu) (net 79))
 (segment (start 175.908 118) (end 182.88 124.972) (width 0.25) (layer F.Cu) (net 79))
 (segment (start 165 118) (end 175.908 118) (width 0.25) (layer F.Cu) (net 79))
 (segment (start 146.05 92.71) (end 146.05 96.05) (width 0.25) (layer F.Cu) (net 78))
 (segment (start 146.05 96.05) (end 166 116) (width 0.25) (layer F.Cu) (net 78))
 (segment (start 185.42 124.972) (end 185.42 128.397) (width 0.25) (layer F.Cu) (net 78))
 (segment (start 176.448 116) (end 185.42 124.972) (width 0.25) (layer F.Cu) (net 78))
 (segment (start 166 116) (end 176.448 116) (width 0.25) (layer F.Cu) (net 78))
 (segment (start 187.96 124.96) (end 187.96 128.397) (width 0.25) (layer F.Cu) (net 77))
 (segment (start 178 115) (end 187.96 124.96) (width 0.25) (layer F.Cu) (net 77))
 (segment (start 167 115) (end 178 115) (width 0.25) (layer F.Cu) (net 77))
 (segment (start 148.59 92.71) (end 148.59 96.59) (width 0.25) (layer F.Cu) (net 77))
 (segment (start 148.59 96.59) (end 167 115) (width 0.25) (layer F.Cu) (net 77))
 (segment (start 151.13 92.71) (end 151.13 96.13) (width 0.25) (layer F.Cu) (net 76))
 (segment (start 151.13 96.13) (end 168 113) (width 0.25) (layer F.Cu) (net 76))
 (segment (start 190.5 126.317798) (end 190.5 128.397) (width 0.25) (layer F.Cu) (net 76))
 (segment (start 177.182202 113) (end 190.5 126.317798) (width 0.25) (layer F.Cu) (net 76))
 (segment (start 168 113) (end 177.182202 113) (width 0.25) (layer F.Cu) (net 76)))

